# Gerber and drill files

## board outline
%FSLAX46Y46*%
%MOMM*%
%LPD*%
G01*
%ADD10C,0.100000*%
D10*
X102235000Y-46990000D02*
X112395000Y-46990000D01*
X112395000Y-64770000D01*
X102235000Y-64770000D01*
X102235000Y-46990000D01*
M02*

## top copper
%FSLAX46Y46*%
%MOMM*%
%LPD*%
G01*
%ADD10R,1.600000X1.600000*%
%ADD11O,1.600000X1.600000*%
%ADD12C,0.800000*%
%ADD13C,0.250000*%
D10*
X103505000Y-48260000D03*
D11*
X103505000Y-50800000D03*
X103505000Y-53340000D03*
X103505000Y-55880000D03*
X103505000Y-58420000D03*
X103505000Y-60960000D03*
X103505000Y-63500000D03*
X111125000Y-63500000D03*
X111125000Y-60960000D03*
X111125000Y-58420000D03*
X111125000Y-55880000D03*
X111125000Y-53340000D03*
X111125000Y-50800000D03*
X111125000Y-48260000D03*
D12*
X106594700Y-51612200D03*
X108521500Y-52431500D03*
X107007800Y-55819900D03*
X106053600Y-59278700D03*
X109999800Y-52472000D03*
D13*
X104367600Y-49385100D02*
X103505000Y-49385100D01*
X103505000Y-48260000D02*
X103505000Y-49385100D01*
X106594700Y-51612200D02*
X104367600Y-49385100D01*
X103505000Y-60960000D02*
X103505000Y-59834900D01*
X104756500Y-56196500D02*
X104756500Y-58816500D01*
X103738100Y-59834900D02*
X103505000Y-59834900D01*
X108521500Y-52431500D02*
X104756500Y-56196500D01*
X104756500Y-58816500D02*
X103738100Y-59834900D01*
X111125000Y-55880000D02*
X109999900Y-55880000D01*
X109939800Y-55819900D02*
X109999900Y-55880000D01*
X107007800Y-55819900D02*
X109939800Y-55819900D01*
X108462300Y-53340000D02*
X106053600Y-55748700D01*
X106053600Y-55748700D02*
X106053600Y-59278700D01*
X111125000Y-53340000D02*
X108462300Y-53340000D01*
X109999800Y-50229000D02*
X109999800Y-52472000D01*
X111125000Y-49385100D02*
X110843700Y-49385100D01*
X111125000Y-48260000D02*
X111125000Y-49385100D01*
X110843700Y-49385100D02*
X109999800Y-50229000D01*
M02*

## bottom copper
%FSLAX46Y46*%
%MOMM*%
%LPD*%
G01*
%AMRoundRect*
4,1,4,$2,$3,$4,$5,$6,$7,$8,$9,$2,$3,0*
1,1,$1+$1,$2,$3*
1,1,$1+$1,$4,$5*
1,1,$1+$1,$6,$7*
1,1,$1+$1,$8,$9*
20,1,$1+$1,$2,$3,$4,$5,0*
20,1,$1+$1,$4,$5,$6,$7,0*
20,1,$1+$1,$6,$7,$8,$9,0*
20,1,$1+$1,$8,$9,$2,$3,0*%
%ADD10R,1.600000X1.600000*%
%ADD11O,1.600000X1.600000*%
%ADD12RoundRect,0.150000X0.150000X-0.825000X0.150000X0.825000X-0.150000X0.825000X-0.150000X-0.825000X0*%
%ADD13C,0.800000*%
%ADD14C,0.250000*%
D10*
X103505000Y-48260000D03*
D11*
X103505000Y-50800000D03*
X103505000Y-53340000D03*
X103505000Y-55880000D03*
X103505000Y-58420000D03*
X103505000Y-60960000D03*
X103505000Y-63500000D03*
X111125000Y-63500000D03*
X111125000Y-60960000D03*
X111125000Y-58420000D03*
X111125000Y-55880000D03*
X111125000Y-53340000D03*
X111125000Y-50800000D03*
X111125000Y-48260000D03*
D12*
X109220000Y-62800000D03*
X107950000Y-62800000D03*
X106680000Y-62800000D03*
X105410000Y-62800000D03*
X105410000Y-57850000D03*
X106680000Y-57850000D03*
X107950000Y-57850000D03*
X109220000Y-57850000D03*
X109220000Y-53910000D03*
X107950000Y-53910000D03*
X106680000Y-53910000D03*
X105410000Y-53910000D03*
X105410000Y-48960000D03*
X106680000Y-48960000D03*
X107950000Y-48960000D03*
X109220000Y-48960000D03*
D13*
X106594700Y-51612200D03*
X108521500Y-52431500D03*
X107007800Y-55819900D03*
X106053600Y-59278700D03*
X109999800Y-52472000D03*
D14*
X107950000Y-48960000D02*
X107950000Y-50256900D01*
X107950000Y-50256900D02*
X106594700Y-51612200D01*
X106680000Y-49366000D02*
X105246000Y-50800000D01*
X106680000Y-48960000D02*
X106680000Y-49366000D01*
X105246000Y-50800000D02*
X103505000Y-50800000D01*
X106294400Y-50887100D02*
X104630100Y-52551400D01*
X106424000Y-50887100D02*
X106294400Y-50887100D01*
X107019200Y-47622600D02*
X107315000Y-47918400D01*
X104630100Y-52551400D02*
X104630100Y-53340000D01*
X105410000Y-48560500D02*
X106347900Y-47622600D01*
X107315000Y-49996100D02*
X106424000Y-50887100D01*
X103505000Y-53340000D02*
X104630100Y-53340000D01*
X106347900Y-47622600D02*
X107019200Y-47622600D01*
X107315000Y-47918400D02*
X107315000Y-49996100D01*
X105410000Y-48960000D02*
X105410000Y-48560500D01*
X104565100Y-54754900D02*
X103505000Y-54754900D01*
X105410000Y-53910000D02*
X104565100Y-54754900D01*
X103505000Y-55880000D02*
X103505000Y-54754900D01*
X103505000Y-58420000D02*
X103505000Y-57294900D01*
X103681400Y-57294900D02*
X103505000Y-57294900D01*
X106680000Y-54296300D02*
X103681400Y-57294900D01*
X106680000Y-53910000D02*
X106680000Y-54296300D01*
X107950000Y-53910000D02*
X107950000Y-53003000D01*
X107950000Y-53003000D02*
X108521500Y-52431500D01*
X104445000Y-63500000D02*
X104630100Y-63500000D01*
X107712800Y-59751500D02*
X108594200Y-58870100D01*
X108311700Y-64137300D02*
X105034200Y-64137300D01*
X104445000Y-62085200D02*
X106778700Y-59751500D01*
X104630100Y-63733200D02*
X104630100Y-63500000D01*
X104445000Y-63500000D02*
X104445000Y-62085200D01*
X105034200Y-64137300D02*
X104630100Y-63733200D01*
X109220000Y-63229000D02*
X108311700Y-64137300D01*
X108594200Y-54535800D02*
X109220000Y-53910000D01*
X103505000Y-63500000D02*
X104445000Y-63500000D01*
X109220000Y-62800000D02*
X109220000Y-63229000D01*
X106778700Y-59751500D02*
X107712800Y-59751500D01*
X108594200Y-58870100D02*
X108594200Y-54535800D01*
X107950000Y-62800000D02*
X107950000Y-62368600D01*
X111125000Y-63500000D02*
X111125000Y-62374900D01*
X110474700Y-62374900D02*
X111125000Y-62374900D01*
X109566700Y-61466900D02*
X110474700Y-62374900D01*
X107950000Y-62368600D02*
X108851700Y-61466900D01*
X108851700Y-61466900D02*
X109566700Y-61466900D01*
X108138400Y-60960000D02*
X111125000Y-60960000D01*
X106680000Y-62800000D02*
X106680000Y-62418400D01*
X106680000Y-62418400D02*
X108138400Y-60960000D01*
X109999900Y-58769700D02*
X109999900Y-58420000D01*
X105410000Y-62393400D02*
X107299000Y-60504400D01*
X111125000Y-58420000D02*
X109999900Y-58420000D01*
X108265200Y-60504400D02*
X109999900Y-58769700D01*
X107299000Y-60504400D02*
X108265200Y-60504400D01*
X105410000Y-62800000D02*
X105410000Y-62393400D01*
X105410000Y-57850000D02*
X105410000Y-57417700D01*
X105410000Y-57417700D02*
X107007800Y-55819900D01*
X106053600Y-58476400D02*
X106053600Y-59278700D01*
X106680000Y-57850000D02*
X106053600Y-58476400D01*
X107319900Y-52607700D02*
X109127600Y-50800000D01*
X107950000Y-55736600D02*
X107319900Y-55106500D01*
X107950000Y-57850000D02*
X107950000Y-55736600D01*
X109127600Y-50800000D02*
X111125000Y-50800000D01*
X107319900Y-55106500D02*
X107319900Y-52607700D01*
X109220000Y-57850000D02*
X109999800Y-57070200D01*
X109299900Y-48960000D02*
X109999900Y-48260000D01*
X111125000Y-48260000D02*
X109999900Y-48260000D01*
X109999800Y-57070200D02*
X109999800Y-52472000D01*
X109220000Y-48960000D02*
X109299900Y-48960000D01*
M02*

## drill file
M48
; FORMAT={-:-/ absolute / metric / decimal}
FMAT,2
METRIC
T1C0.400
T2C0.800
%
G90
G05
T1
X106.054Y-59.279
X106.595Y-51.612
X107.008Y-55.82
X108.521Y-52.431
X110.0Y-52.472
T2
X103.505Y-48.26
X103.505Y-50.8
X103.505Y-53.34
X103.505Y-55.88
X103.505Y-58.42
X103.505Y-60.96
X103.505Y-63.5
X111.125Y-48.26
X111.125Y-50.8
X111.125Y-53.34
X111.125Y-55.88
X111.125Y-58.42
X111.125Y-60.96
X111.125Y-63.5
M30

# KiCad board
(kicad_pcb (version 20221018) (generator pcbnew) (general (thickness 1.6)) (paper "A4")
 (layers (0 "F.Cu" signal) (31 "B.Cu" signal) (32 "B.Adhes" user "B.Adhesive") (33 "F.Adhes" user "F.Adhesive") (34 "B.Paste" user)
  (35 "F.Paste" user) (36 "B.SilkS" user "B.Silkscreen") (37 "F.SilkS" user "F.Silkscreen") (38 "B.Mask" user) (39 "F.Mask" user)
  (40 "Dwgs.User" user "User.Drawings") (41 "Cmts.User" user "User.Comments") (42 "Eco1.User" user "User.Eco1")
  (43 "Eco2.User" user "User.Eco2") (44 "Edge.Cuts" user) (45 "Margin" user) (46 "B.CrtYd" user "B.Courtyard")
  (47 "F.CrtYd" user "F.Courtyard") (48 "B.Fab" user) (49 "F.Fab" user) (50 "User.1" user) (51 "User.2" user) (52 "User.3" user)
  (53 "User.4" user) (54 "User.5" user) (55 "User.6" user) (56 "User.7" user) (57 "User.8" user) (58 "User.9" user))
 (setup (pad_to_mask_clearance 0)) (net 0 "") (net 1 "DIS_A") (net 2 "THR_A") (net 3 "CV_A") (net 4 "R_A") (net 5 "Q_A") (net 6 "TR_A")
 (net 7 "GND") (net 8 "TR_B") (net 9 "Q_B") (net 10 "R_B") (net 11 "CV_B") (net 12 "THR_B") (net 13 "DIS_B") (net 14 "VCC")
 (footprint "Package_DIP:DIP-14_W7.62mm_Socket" (layer "F.Cu") (at 103.505 48.26)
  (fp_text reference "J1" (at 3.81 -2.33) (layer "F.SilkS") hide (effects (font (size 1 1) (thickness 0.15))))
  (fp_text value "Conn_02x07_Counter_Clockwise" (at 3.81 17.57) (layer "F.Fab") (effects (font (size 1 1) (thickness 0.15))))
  (pad "1" thru_hole rect (at 0 0) (size 1.6 1.6) (drill 0.8) (layers "*.Cu" "*.Mask") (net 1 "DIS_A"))
  (pad "2" thru_hole oval (at 0 2.54) (size 1.6 1.6) (drill 0.8) (layers "*.Cu" "*.Mask") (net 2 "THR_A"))
  (pad "3" thru_hole oval (at 0 5.08) (size 1.6 1.6) (drill 0.8) (layers "*.Cu" "*.Mask") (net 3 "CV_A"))
  (pad "4" thru_hole oval (at 0 7.62) (size 1.6 1.6) (drill 0.8) (layers "*.Cu" "*.Mask") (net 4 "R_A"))
  (pad "5" thru_hole oval (at 0 10.16) (size 1.6 1.6) (drill 0.8) (layers "*.Cu" "*.Mask") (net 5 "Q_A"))
  (pad "6" thru_hole oval (at 0 12.7) (size 1.6 1.6) (drill 0.8) (layers "*.Cu" "*.Mask") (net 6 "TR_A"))
  (pad "7" thru_hole oval (at 0 15.24) (size 1.6 1.6) (drill 0.8) (layers "*.Cu" "*.Mask") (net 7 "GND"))
  (pad "8" thru_hole oval (at 7.62 15.24) (size 1.6 1.6) (drill 0.8) (layers "*.Cu" "*.Mask") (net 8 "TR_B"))
  (pad "9" thru_hole oval (at 7.62 12.7) (size 1.6 1.6) (drill 0.8) (layers "*.Cu" "*.Mask") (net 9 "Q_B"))
  (pad "10" thru_hole oval (at 7.62 10.16) (size 1.6 1.6) (drill 0.8) (layers "*.Cu" "*.Mask") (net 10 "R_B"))
  (pad "11" thru_hole oval (at 7.62 7.62) (size 1.6 1.6) (drill 0.8) (layers "*.Cu" "*.Mask") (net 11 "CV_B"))
  (pad "12" thru_hole oval (at 7.62 5.08) (size 1.6 1.6) (drill 0.8) (layers "*.Cu" "*.Mask") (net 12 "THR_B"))
  (pad "13" thru_hole oval (at 7.62 2.54) (size 1.6 1.6) (drill 0.8) (layers "*.Cu" "*.Mask") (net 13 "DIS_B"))
  (pad "14" thru_hole oval (at 7.62 0) (size 1.6 1.6) (drill 0.8) (layers "*.Cu" "*.Mask") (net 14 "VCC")))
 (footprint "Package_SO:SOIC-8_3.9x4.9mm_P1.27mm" (layer "B.Cu") (at 107.315 60.325 90)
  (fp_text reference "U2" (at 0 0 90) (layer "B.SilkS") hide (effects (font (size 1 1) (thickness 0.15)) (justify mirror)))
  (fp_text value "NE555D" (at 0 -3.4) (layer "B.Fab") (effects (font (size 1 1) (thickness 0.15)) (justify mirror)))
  (pad "1" smd roundrect (at -2.475 1.905 90) (size 1.95 0.6) (layers "B.Cu" "B.Paste" "B.Mask") (roundrect_rratio 0.25) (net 7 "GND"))
  (pad "2" smd roundrect (at -2.475 0.635 90) (size 1.95 0.6) (layers "B.Cu" "B.Paste" "B.Mask") (roundrect_rratio 0.25) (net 8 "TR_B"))
  (pad "3" smd roundrect (at -2.475 -0.635 90) (size 1.95 0.6) (layers "B.Cu" "B.Paste" "B.Mask") (roundrect_rratio 0.25) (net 9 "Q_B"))
  (pad "4" smd roundrect (at -2.475 -1.905 90) (size 1.95 0.6) (layers "B.Cu" "B.Paste" "B.Mask") (roundrect_rratio 0.25) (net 10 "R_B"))
  (pad "5" smd roundrect (at 2.475 -1.905 90) (size 1.95 0.6) (layers "B.Cu" "B.Paste" "B.Mask") (roundrect_rratio 0.25) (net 11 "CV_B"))
  (pad "6" smd roundrect (at 2.475 -0.635 90) (size 1.95 0.6) (layers "B.Cu" "B.Paste" "B.Mask") (roundrect_rratio 0.25) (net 12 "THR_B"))
  (pad "7" smd roundrect (at 2.475 0.635 90) (size 1.95 0.6) (layers "B.Cu" "B.Paste" "B.Mask") (roundrect_rratio 0.25) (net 13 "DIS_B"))
  (pad "8" smd roundrect (at 2.475 1.905 90) (size 1.95 0.6) (layers "B.Cu" "B.Paste" "B.Mask") (roundrect_rratio 0.25) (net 14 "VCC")))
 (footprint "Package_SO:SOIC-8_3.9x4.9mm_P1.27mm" (layer "B.Cu") (at 107.315 51.435 90)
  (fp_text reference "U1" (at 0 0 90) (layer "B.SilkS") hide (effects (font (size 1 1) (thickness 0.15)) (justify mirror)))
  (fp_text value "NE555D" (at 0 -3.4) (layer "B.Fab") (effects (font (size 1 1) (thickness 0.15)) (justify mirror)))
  (pad "1" smd roundrect (at -2.475 1.905 90) (size 1.95 0.6) (layers "B.Cu" "B.Paste" "B.Mask") (roundrect_rratio 0.25) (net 7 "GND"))
  (pad "2" smd roundrect (at -2.475 0.635 90) (size 1.95 0.6) (layers "B.Cu" "B.Paste" "B.Mask") (roundrect_rratio 0.25) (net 6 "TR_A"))
  (pad "3" smd roundrect (at -2.475 -0.635 90) (size 1.95 0.6) (layers "B.Cu" "B.Paste" "B.Mask") (roundrect_rratio 0.25) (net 5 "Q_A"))
  (pad "4" smd roundrect (at -2.475 -1.905 90) (size 1.95 0.6) (layers "B.Cu" "B.Paste" "B.Mask") (roundrect_rratio 0.25) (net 4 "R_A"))
  (pad "5" smd roundrect (at 2.475 -1.905 90) (size 1.95 0.6) (layers "B.Cu" "B.Paste" "B.Mask") (roundrect_rratio 0.25) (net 3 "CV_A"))
  (pad "6" smd roundrect (at 2.475 -0.635 90) (size 1.95 0.6) (layers "B.Cu" "B.Paste" "B.Mask") (roundrect_rratio 0.25) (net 2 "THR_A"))
  (pad "7" smd roundrect (at 2.475 0.635 90) (size 1.95 0.6) (layers "B.Cu" "B.Paste" "B.Mask") (roundrect_rratio 0.25) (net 1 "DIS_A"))
  (pad "8" smd roundrect (at 2.475 1.905 90) (size 1.95 0.6) (layers "B.Cu" "B.Paste" "B.Mask") (roundrect_rratio 0.25) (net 14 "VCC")))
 (gr_rect (start 102.235 46.99) (end 112.395 64.77) (stroke (width 0.1) (type default)) (fill none) (layer "Edge.Cuts"))
 (segment (start 104.3676 49.3851) (end 103.505 49.3851) (width 0.25) (layer "F.Cu") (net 1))
 (segment (start 103.505 48.26) (end 103.505 49.3851) (width 0.25) (layer "F.Cu") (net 1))
 (segment (start 106.5947 51.6122) (end 104.3676 49.3851) (width 0.25) (layer "F.Cu") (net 1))
 (via (at 106.5947 51.6122) (size 0.8) (drill 0.4) (layers "F.Cu" "B.Cu") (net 1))
 (segment (start 107.95 48.96) (end 107.95 50.2569) (width 0.25) (layer "B.Cu") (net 1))
 (segment (start 107.95 50.2569) (end 106.5947 51.6122) (width 0.25) (layer "B.Cu") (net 1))
 (segment (start 106.68 49.366) (end 105.246 50.8) (width 0.25) (layer "B.Cu") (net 2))
 (segment (start 106.68 48.96) (end 106.68 49.366) (width 0.25) (layer "B.Cu") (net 2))
 (segment (start 105.246 50.8) (end 103.505 50.8) (width 0.25) (layer "B.Cu") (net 2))
 (segment (start 106.2944 50.8871) (end 104.6301 52.5514) (width 0.25) (layer "B.Cu") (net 3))
 (segment (start 106.424 50.8871) (end 106.2944 50.8871) (width 0.25) (layer "B.Cu") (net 3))
 (segment (start 107.0192 47.6226) (end 107.315 47.9184) (width 0.25) (layer "B.Cu") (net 3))
 (segment (start 104.6301 52.5514) (end 104.6301 53.34) (width 0.25) (layer "B.Cu") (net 3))
 (segment (start 105.41 48.5605) (end 106.3479 47.6226) (width 0.25) (layer "B.Cu") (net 3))
 (segment (start 107.315 49.9961) (end 106.424 50.8871) (width 0.25) (layer "B.Cu") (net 3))
 (segment (start 103.505 53.34) (end 104.6301 53.34) (width 0.25) (layer "B.Cu") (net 3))
 (segment (start 106.3479 47.6226) (end 107.0192 47.6226) (width 0.25) (layer "B.Cu") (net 3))
 (segment (start 107.315 47.9184) (end 107.315 49.9961) (width 0.25) (layer "B.Cu") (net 3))
 (segment (start 105.41 48.96) (end 105.41 48.5605) (width 0.25) (layer "B.Cu") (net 3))
 (segment (start 104.5651 54.7549) (end 103.505 54.7549) (width 0.25) (layer "B.Cu") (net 4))
 (segment (start 105.41 53.91) (end 104.5651 54.7549) (width 0.25) (layer "B.Cu") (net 4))
 (segment (start 103.505 55.88) (end 103.505 54.7549) (width 0.25) (layer "B.Cu") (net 4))
 (segment (start 103.505 58.42) (end 103.505 57.2949) (width 0.25) (layer "B.Cu") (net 5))
 (segment (start 103.6814 57.2949) (end 103.505 57.2949) (width 0.25) (layer "B.Cu") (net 5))
 (segment (start 106.68 54.2963) (end 103.6814 57.2949) (width 0.25) (layer "B.Cu") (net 5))
 (segment (start 106.68 53.91) (end 106.68 54.2963) (width 0.25) (layer "B.Cu") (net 5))
 (segment (start 103.505 60.96) (end 103.505 59.8349) (width 0.25) (layer "F.Cu") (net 6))
 (segment (start 104.7565 56.1965) (end 104.7565 58.8165) (width 0.25) (layer "F.Cu") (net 6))
 (segment (start 103.7381 59.8349) (end 103.505 59.8349) (width 0.25) (layer "F.Cu") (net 6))
 (segment (start 108.5215 52.4315) (end 104.7565 56.1965) (width 0.25) (layer "F.Cu") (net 6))
 (segment (start 104.7565 58.8165) (end 103.7381 59.8349) (width 0.25) (layer "F.Cu") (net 6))
 (via (at 108.5215 52.4315) (size 0.8) (drill 0.4) (layers "F.Cu" "B.Cu") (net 6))
 (segment (start 107.95 53.91) (end 107.95 53.003) (width 0.25) (layer "B.Cu") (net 6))
 (segment (start 107.95 53.003) (end 108.5215 52.4315) (width 0.25) (layer "B.Cu") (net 6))
 (segment (start 104.445 63.5) (end 104.6301 63.5) (width 0.25) (layer "B.Cu") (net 7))
 (segment (start 107.7128 59.7515) (end 108.5942 58.8701) (width 0.25) (layer "B.Cu") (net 7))
 (segment (start 108.3117 64.1373) (end 105.0342 64.1373) (width 0.25) (layer "B.Cu") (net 7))
 (segment (start 104.445 62.0852) (end 106.7787 59.7515) (width 0.25) (layer "B.Cu") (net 7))
 (segment (start 104.6301 63.7332) (end 104.6301 63.5) (width 0.25) (layer "B.Cu") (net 7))
 (segment (start 104.445 63.5) (end 104.445 62.0852) (width 0.25) (layer "B.Cu") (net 7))
 (segment (start 105.0342 64.1373) (end 104.6301 63.7332) (width 0.25) (layer "B.Cu") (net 7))
 (segment (start 109.22 63.229) (end 108.3117 64.1373) (width 0.25) (layer "B.Cu") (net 7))
 (segment (start 108.5942 54.5358) (end 109.22 53.91) (width 0.25) (layer "B.Cu") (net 7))
 (segment (start 103.505 63.5) (end 104.445 63.5) (width 0.25) (layer "B.Cu") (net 7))
 (segment (start 109.22 62.8) (end 109.22 63.229) (width 0.25) (layer "B.Cu") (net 7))
 (segment (start 106.7787 59.7515) (end 107.7128 59.7515) (width 0.25) (layer "B.Cu") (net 7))
 (segment (start 108.5942 58.8701) (end 108.5942 54.5358) (width 0.25) (layer "B.Cu") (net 7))
 (segment (start 107.95 62.8) (end 107.95 62.3686) (width 0.25) (layer "B.Cu") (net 8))
 (segment (start 111.125 63.5) (end 111.125 62.3749) (width 0.25) (layer "B.Cu") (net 8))
 (segment (start 110.4747 62.3749) (end 111.125 62.3749) (width 0.25) (layer "B.Cu") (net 8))
 (segment (start 109.5667 61.4669) (end 110.4747 62.3749) (width 0.25) (layer "B.Cu") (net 8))
 (segment (start 107.95 62.3686) (end 108.8517 61.4669) (width 0.25) (layer "B.Cu") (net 8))
 (segment (start 108.8517 61.4669) (end 109.5667 61.4669) (width 0.25) (layer "B.Cu") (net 8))
 (segment (start 108.1384 60.96) (end 111.125 60.96) (width 0.25) (layer "B.Cu") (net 9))
 (segment (start 106.68 62.8) (end 106.68 62.4184) (width 0.25) (layer "B.Cu") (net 9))
 (segment (start 106.68 62.4184) (end 108.1384 60.96) (width 0.25) (layer "B.Cu") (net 9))
 (segment (start 109.9999 58.7697) (end 109.9999 58.42) (width 0.25) (layer "B.Cu") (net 10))
 (segment (start 105.41 62.3934) (end 107.299 60.5044) (width 0.25) (layer "B.Cu") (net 10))
 (segment (start 111.125 58.42) (end 109.9999 58.42) (width 0.25) (layer "B.Cu") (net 10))
 (segment (start 108.2652 60.5044) (end 109.9999 58.7697) (width 0.25) (layer "B.Cu") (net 10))
 (segment (start 107.299 60.5044) (end 108.2652 60.5044) (width 0.25) (layer "B.Cu") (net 10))
 (segment (start 105.41 62.8) (end 105.41 62.3934) (width 0.25) (layer "B.Cu") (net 10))
 (segment (start 111.125 55.88) (end 109.9999 55.88) (width 0.25) (layer "F.Cu") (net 11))
 (segment (start 109.9398 55.8199) (end 109.9999 55.88) (width 0.25) (layer "F.Cu") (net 11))
 (segment (start 107.0078 55.8199) (end 109.9398 55.8199) (width 0.25) (layer "F.Cu") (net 11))
 (via (at 107.0078 55.8199) (size 0.8) (drill 0.4) (layers "F.Cu" "B.Cu") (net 11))
 (segment (start 105.41 57.85) (end 105.41 57.4177) (width 0.25) (layer "B.Cu") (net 11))
 (segment (start 105.41 57.4177) (end 107.0078 55.8199) (width 0.25) (layer "B.Cu") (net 11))
 (segment (start 108.4623 53.34) (end 106.0536 55.7487) (width 0.25) (layer "F.Cu") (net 12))
 (segment (start 106.0536 55.7487) (end 106.0536 59.2787) (width 0.25) (layer "F.Cu") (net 12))
 (segment (start 111.125 53.34) (end 108.4623 53.34) (width 0.25) (layer "F.Cu") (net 12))
 (via (at 106.0536 59.2787) (size 0.8) (drill 0.4) (layers "F.Cu" "B.Cu") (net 12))
 (segment (start 106.0536 58.4764) (end 106.0536 59.2787) (width 0.25) (layer "B.Cu") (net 12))
 (segment (start 106.68 57.85) (end 106.0536 58.4764) (width 0.25) (layer "B.Cu") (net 12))
 (segment (start 107.3199 52.6077) (end 109.1276 50.8) (width 0.25) (layer "B.Cu") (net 13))
 (segment (start 107.95 55.7366) (end 107.3199 55.1065) (width 0.25) (layer "B.Cu") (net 13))
 (segment (start 107.95 57.85) (end 107.95 55.7366) (width 0.25) (layer "B.Cu") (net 13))
 (segment (start 109.1276 50.8) (end 111.125 50.8) (width 0.25) (layer "B.Cu") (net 13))
 (segment (start 107.3199 55.1065) (end 107.3199 52.6077) (width 0.25) (layer "B.Cu") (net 13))
 (segment (start 109.9998 50.229) (end 109.9998 52.472) (width 0.25) (layer "F.Cu") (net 14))
 (segment (start 111.125 49.3851) (end 110.8437 49.3851) (width 0.25) (layer "F.Cu") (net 14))
 (segment (start 111.125 48.26) (end 111.125 49.3851) (width 0.25) (layer "F.Cu") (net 14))
 (segment (start 110.8437 49.3851) (end 109.9998 50.229) (width 0.25) (layer "F.Cu") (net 14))
 (via (at 109.9998 52.472) (size 0.8) (drill 0.4) (layers "F.Cu" "B.Cu") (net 14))
 (segment (start 109.22 57.85) (end 109.9998 57.0702) (width 0.25) (layer "B.Cu") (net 14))
 (segment (start 109.2999 48.96) (end 109.9999 48.26) (width 0.25) (layer "B.Cu") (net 14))
 (segment (start 111.125 48.26) (end 109.9999 48.26) (width 0.25) (layer "B.Cu") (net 14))
 (segment (start 109.9998 57.0702) (end 109.9998 52.472) (width 0.25) (layer "B.Cu") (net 14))
 (segment (start 109.22 48.96) (end 109.2999 48.96) (width 0.25) (layer "B.Cu") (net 14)))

